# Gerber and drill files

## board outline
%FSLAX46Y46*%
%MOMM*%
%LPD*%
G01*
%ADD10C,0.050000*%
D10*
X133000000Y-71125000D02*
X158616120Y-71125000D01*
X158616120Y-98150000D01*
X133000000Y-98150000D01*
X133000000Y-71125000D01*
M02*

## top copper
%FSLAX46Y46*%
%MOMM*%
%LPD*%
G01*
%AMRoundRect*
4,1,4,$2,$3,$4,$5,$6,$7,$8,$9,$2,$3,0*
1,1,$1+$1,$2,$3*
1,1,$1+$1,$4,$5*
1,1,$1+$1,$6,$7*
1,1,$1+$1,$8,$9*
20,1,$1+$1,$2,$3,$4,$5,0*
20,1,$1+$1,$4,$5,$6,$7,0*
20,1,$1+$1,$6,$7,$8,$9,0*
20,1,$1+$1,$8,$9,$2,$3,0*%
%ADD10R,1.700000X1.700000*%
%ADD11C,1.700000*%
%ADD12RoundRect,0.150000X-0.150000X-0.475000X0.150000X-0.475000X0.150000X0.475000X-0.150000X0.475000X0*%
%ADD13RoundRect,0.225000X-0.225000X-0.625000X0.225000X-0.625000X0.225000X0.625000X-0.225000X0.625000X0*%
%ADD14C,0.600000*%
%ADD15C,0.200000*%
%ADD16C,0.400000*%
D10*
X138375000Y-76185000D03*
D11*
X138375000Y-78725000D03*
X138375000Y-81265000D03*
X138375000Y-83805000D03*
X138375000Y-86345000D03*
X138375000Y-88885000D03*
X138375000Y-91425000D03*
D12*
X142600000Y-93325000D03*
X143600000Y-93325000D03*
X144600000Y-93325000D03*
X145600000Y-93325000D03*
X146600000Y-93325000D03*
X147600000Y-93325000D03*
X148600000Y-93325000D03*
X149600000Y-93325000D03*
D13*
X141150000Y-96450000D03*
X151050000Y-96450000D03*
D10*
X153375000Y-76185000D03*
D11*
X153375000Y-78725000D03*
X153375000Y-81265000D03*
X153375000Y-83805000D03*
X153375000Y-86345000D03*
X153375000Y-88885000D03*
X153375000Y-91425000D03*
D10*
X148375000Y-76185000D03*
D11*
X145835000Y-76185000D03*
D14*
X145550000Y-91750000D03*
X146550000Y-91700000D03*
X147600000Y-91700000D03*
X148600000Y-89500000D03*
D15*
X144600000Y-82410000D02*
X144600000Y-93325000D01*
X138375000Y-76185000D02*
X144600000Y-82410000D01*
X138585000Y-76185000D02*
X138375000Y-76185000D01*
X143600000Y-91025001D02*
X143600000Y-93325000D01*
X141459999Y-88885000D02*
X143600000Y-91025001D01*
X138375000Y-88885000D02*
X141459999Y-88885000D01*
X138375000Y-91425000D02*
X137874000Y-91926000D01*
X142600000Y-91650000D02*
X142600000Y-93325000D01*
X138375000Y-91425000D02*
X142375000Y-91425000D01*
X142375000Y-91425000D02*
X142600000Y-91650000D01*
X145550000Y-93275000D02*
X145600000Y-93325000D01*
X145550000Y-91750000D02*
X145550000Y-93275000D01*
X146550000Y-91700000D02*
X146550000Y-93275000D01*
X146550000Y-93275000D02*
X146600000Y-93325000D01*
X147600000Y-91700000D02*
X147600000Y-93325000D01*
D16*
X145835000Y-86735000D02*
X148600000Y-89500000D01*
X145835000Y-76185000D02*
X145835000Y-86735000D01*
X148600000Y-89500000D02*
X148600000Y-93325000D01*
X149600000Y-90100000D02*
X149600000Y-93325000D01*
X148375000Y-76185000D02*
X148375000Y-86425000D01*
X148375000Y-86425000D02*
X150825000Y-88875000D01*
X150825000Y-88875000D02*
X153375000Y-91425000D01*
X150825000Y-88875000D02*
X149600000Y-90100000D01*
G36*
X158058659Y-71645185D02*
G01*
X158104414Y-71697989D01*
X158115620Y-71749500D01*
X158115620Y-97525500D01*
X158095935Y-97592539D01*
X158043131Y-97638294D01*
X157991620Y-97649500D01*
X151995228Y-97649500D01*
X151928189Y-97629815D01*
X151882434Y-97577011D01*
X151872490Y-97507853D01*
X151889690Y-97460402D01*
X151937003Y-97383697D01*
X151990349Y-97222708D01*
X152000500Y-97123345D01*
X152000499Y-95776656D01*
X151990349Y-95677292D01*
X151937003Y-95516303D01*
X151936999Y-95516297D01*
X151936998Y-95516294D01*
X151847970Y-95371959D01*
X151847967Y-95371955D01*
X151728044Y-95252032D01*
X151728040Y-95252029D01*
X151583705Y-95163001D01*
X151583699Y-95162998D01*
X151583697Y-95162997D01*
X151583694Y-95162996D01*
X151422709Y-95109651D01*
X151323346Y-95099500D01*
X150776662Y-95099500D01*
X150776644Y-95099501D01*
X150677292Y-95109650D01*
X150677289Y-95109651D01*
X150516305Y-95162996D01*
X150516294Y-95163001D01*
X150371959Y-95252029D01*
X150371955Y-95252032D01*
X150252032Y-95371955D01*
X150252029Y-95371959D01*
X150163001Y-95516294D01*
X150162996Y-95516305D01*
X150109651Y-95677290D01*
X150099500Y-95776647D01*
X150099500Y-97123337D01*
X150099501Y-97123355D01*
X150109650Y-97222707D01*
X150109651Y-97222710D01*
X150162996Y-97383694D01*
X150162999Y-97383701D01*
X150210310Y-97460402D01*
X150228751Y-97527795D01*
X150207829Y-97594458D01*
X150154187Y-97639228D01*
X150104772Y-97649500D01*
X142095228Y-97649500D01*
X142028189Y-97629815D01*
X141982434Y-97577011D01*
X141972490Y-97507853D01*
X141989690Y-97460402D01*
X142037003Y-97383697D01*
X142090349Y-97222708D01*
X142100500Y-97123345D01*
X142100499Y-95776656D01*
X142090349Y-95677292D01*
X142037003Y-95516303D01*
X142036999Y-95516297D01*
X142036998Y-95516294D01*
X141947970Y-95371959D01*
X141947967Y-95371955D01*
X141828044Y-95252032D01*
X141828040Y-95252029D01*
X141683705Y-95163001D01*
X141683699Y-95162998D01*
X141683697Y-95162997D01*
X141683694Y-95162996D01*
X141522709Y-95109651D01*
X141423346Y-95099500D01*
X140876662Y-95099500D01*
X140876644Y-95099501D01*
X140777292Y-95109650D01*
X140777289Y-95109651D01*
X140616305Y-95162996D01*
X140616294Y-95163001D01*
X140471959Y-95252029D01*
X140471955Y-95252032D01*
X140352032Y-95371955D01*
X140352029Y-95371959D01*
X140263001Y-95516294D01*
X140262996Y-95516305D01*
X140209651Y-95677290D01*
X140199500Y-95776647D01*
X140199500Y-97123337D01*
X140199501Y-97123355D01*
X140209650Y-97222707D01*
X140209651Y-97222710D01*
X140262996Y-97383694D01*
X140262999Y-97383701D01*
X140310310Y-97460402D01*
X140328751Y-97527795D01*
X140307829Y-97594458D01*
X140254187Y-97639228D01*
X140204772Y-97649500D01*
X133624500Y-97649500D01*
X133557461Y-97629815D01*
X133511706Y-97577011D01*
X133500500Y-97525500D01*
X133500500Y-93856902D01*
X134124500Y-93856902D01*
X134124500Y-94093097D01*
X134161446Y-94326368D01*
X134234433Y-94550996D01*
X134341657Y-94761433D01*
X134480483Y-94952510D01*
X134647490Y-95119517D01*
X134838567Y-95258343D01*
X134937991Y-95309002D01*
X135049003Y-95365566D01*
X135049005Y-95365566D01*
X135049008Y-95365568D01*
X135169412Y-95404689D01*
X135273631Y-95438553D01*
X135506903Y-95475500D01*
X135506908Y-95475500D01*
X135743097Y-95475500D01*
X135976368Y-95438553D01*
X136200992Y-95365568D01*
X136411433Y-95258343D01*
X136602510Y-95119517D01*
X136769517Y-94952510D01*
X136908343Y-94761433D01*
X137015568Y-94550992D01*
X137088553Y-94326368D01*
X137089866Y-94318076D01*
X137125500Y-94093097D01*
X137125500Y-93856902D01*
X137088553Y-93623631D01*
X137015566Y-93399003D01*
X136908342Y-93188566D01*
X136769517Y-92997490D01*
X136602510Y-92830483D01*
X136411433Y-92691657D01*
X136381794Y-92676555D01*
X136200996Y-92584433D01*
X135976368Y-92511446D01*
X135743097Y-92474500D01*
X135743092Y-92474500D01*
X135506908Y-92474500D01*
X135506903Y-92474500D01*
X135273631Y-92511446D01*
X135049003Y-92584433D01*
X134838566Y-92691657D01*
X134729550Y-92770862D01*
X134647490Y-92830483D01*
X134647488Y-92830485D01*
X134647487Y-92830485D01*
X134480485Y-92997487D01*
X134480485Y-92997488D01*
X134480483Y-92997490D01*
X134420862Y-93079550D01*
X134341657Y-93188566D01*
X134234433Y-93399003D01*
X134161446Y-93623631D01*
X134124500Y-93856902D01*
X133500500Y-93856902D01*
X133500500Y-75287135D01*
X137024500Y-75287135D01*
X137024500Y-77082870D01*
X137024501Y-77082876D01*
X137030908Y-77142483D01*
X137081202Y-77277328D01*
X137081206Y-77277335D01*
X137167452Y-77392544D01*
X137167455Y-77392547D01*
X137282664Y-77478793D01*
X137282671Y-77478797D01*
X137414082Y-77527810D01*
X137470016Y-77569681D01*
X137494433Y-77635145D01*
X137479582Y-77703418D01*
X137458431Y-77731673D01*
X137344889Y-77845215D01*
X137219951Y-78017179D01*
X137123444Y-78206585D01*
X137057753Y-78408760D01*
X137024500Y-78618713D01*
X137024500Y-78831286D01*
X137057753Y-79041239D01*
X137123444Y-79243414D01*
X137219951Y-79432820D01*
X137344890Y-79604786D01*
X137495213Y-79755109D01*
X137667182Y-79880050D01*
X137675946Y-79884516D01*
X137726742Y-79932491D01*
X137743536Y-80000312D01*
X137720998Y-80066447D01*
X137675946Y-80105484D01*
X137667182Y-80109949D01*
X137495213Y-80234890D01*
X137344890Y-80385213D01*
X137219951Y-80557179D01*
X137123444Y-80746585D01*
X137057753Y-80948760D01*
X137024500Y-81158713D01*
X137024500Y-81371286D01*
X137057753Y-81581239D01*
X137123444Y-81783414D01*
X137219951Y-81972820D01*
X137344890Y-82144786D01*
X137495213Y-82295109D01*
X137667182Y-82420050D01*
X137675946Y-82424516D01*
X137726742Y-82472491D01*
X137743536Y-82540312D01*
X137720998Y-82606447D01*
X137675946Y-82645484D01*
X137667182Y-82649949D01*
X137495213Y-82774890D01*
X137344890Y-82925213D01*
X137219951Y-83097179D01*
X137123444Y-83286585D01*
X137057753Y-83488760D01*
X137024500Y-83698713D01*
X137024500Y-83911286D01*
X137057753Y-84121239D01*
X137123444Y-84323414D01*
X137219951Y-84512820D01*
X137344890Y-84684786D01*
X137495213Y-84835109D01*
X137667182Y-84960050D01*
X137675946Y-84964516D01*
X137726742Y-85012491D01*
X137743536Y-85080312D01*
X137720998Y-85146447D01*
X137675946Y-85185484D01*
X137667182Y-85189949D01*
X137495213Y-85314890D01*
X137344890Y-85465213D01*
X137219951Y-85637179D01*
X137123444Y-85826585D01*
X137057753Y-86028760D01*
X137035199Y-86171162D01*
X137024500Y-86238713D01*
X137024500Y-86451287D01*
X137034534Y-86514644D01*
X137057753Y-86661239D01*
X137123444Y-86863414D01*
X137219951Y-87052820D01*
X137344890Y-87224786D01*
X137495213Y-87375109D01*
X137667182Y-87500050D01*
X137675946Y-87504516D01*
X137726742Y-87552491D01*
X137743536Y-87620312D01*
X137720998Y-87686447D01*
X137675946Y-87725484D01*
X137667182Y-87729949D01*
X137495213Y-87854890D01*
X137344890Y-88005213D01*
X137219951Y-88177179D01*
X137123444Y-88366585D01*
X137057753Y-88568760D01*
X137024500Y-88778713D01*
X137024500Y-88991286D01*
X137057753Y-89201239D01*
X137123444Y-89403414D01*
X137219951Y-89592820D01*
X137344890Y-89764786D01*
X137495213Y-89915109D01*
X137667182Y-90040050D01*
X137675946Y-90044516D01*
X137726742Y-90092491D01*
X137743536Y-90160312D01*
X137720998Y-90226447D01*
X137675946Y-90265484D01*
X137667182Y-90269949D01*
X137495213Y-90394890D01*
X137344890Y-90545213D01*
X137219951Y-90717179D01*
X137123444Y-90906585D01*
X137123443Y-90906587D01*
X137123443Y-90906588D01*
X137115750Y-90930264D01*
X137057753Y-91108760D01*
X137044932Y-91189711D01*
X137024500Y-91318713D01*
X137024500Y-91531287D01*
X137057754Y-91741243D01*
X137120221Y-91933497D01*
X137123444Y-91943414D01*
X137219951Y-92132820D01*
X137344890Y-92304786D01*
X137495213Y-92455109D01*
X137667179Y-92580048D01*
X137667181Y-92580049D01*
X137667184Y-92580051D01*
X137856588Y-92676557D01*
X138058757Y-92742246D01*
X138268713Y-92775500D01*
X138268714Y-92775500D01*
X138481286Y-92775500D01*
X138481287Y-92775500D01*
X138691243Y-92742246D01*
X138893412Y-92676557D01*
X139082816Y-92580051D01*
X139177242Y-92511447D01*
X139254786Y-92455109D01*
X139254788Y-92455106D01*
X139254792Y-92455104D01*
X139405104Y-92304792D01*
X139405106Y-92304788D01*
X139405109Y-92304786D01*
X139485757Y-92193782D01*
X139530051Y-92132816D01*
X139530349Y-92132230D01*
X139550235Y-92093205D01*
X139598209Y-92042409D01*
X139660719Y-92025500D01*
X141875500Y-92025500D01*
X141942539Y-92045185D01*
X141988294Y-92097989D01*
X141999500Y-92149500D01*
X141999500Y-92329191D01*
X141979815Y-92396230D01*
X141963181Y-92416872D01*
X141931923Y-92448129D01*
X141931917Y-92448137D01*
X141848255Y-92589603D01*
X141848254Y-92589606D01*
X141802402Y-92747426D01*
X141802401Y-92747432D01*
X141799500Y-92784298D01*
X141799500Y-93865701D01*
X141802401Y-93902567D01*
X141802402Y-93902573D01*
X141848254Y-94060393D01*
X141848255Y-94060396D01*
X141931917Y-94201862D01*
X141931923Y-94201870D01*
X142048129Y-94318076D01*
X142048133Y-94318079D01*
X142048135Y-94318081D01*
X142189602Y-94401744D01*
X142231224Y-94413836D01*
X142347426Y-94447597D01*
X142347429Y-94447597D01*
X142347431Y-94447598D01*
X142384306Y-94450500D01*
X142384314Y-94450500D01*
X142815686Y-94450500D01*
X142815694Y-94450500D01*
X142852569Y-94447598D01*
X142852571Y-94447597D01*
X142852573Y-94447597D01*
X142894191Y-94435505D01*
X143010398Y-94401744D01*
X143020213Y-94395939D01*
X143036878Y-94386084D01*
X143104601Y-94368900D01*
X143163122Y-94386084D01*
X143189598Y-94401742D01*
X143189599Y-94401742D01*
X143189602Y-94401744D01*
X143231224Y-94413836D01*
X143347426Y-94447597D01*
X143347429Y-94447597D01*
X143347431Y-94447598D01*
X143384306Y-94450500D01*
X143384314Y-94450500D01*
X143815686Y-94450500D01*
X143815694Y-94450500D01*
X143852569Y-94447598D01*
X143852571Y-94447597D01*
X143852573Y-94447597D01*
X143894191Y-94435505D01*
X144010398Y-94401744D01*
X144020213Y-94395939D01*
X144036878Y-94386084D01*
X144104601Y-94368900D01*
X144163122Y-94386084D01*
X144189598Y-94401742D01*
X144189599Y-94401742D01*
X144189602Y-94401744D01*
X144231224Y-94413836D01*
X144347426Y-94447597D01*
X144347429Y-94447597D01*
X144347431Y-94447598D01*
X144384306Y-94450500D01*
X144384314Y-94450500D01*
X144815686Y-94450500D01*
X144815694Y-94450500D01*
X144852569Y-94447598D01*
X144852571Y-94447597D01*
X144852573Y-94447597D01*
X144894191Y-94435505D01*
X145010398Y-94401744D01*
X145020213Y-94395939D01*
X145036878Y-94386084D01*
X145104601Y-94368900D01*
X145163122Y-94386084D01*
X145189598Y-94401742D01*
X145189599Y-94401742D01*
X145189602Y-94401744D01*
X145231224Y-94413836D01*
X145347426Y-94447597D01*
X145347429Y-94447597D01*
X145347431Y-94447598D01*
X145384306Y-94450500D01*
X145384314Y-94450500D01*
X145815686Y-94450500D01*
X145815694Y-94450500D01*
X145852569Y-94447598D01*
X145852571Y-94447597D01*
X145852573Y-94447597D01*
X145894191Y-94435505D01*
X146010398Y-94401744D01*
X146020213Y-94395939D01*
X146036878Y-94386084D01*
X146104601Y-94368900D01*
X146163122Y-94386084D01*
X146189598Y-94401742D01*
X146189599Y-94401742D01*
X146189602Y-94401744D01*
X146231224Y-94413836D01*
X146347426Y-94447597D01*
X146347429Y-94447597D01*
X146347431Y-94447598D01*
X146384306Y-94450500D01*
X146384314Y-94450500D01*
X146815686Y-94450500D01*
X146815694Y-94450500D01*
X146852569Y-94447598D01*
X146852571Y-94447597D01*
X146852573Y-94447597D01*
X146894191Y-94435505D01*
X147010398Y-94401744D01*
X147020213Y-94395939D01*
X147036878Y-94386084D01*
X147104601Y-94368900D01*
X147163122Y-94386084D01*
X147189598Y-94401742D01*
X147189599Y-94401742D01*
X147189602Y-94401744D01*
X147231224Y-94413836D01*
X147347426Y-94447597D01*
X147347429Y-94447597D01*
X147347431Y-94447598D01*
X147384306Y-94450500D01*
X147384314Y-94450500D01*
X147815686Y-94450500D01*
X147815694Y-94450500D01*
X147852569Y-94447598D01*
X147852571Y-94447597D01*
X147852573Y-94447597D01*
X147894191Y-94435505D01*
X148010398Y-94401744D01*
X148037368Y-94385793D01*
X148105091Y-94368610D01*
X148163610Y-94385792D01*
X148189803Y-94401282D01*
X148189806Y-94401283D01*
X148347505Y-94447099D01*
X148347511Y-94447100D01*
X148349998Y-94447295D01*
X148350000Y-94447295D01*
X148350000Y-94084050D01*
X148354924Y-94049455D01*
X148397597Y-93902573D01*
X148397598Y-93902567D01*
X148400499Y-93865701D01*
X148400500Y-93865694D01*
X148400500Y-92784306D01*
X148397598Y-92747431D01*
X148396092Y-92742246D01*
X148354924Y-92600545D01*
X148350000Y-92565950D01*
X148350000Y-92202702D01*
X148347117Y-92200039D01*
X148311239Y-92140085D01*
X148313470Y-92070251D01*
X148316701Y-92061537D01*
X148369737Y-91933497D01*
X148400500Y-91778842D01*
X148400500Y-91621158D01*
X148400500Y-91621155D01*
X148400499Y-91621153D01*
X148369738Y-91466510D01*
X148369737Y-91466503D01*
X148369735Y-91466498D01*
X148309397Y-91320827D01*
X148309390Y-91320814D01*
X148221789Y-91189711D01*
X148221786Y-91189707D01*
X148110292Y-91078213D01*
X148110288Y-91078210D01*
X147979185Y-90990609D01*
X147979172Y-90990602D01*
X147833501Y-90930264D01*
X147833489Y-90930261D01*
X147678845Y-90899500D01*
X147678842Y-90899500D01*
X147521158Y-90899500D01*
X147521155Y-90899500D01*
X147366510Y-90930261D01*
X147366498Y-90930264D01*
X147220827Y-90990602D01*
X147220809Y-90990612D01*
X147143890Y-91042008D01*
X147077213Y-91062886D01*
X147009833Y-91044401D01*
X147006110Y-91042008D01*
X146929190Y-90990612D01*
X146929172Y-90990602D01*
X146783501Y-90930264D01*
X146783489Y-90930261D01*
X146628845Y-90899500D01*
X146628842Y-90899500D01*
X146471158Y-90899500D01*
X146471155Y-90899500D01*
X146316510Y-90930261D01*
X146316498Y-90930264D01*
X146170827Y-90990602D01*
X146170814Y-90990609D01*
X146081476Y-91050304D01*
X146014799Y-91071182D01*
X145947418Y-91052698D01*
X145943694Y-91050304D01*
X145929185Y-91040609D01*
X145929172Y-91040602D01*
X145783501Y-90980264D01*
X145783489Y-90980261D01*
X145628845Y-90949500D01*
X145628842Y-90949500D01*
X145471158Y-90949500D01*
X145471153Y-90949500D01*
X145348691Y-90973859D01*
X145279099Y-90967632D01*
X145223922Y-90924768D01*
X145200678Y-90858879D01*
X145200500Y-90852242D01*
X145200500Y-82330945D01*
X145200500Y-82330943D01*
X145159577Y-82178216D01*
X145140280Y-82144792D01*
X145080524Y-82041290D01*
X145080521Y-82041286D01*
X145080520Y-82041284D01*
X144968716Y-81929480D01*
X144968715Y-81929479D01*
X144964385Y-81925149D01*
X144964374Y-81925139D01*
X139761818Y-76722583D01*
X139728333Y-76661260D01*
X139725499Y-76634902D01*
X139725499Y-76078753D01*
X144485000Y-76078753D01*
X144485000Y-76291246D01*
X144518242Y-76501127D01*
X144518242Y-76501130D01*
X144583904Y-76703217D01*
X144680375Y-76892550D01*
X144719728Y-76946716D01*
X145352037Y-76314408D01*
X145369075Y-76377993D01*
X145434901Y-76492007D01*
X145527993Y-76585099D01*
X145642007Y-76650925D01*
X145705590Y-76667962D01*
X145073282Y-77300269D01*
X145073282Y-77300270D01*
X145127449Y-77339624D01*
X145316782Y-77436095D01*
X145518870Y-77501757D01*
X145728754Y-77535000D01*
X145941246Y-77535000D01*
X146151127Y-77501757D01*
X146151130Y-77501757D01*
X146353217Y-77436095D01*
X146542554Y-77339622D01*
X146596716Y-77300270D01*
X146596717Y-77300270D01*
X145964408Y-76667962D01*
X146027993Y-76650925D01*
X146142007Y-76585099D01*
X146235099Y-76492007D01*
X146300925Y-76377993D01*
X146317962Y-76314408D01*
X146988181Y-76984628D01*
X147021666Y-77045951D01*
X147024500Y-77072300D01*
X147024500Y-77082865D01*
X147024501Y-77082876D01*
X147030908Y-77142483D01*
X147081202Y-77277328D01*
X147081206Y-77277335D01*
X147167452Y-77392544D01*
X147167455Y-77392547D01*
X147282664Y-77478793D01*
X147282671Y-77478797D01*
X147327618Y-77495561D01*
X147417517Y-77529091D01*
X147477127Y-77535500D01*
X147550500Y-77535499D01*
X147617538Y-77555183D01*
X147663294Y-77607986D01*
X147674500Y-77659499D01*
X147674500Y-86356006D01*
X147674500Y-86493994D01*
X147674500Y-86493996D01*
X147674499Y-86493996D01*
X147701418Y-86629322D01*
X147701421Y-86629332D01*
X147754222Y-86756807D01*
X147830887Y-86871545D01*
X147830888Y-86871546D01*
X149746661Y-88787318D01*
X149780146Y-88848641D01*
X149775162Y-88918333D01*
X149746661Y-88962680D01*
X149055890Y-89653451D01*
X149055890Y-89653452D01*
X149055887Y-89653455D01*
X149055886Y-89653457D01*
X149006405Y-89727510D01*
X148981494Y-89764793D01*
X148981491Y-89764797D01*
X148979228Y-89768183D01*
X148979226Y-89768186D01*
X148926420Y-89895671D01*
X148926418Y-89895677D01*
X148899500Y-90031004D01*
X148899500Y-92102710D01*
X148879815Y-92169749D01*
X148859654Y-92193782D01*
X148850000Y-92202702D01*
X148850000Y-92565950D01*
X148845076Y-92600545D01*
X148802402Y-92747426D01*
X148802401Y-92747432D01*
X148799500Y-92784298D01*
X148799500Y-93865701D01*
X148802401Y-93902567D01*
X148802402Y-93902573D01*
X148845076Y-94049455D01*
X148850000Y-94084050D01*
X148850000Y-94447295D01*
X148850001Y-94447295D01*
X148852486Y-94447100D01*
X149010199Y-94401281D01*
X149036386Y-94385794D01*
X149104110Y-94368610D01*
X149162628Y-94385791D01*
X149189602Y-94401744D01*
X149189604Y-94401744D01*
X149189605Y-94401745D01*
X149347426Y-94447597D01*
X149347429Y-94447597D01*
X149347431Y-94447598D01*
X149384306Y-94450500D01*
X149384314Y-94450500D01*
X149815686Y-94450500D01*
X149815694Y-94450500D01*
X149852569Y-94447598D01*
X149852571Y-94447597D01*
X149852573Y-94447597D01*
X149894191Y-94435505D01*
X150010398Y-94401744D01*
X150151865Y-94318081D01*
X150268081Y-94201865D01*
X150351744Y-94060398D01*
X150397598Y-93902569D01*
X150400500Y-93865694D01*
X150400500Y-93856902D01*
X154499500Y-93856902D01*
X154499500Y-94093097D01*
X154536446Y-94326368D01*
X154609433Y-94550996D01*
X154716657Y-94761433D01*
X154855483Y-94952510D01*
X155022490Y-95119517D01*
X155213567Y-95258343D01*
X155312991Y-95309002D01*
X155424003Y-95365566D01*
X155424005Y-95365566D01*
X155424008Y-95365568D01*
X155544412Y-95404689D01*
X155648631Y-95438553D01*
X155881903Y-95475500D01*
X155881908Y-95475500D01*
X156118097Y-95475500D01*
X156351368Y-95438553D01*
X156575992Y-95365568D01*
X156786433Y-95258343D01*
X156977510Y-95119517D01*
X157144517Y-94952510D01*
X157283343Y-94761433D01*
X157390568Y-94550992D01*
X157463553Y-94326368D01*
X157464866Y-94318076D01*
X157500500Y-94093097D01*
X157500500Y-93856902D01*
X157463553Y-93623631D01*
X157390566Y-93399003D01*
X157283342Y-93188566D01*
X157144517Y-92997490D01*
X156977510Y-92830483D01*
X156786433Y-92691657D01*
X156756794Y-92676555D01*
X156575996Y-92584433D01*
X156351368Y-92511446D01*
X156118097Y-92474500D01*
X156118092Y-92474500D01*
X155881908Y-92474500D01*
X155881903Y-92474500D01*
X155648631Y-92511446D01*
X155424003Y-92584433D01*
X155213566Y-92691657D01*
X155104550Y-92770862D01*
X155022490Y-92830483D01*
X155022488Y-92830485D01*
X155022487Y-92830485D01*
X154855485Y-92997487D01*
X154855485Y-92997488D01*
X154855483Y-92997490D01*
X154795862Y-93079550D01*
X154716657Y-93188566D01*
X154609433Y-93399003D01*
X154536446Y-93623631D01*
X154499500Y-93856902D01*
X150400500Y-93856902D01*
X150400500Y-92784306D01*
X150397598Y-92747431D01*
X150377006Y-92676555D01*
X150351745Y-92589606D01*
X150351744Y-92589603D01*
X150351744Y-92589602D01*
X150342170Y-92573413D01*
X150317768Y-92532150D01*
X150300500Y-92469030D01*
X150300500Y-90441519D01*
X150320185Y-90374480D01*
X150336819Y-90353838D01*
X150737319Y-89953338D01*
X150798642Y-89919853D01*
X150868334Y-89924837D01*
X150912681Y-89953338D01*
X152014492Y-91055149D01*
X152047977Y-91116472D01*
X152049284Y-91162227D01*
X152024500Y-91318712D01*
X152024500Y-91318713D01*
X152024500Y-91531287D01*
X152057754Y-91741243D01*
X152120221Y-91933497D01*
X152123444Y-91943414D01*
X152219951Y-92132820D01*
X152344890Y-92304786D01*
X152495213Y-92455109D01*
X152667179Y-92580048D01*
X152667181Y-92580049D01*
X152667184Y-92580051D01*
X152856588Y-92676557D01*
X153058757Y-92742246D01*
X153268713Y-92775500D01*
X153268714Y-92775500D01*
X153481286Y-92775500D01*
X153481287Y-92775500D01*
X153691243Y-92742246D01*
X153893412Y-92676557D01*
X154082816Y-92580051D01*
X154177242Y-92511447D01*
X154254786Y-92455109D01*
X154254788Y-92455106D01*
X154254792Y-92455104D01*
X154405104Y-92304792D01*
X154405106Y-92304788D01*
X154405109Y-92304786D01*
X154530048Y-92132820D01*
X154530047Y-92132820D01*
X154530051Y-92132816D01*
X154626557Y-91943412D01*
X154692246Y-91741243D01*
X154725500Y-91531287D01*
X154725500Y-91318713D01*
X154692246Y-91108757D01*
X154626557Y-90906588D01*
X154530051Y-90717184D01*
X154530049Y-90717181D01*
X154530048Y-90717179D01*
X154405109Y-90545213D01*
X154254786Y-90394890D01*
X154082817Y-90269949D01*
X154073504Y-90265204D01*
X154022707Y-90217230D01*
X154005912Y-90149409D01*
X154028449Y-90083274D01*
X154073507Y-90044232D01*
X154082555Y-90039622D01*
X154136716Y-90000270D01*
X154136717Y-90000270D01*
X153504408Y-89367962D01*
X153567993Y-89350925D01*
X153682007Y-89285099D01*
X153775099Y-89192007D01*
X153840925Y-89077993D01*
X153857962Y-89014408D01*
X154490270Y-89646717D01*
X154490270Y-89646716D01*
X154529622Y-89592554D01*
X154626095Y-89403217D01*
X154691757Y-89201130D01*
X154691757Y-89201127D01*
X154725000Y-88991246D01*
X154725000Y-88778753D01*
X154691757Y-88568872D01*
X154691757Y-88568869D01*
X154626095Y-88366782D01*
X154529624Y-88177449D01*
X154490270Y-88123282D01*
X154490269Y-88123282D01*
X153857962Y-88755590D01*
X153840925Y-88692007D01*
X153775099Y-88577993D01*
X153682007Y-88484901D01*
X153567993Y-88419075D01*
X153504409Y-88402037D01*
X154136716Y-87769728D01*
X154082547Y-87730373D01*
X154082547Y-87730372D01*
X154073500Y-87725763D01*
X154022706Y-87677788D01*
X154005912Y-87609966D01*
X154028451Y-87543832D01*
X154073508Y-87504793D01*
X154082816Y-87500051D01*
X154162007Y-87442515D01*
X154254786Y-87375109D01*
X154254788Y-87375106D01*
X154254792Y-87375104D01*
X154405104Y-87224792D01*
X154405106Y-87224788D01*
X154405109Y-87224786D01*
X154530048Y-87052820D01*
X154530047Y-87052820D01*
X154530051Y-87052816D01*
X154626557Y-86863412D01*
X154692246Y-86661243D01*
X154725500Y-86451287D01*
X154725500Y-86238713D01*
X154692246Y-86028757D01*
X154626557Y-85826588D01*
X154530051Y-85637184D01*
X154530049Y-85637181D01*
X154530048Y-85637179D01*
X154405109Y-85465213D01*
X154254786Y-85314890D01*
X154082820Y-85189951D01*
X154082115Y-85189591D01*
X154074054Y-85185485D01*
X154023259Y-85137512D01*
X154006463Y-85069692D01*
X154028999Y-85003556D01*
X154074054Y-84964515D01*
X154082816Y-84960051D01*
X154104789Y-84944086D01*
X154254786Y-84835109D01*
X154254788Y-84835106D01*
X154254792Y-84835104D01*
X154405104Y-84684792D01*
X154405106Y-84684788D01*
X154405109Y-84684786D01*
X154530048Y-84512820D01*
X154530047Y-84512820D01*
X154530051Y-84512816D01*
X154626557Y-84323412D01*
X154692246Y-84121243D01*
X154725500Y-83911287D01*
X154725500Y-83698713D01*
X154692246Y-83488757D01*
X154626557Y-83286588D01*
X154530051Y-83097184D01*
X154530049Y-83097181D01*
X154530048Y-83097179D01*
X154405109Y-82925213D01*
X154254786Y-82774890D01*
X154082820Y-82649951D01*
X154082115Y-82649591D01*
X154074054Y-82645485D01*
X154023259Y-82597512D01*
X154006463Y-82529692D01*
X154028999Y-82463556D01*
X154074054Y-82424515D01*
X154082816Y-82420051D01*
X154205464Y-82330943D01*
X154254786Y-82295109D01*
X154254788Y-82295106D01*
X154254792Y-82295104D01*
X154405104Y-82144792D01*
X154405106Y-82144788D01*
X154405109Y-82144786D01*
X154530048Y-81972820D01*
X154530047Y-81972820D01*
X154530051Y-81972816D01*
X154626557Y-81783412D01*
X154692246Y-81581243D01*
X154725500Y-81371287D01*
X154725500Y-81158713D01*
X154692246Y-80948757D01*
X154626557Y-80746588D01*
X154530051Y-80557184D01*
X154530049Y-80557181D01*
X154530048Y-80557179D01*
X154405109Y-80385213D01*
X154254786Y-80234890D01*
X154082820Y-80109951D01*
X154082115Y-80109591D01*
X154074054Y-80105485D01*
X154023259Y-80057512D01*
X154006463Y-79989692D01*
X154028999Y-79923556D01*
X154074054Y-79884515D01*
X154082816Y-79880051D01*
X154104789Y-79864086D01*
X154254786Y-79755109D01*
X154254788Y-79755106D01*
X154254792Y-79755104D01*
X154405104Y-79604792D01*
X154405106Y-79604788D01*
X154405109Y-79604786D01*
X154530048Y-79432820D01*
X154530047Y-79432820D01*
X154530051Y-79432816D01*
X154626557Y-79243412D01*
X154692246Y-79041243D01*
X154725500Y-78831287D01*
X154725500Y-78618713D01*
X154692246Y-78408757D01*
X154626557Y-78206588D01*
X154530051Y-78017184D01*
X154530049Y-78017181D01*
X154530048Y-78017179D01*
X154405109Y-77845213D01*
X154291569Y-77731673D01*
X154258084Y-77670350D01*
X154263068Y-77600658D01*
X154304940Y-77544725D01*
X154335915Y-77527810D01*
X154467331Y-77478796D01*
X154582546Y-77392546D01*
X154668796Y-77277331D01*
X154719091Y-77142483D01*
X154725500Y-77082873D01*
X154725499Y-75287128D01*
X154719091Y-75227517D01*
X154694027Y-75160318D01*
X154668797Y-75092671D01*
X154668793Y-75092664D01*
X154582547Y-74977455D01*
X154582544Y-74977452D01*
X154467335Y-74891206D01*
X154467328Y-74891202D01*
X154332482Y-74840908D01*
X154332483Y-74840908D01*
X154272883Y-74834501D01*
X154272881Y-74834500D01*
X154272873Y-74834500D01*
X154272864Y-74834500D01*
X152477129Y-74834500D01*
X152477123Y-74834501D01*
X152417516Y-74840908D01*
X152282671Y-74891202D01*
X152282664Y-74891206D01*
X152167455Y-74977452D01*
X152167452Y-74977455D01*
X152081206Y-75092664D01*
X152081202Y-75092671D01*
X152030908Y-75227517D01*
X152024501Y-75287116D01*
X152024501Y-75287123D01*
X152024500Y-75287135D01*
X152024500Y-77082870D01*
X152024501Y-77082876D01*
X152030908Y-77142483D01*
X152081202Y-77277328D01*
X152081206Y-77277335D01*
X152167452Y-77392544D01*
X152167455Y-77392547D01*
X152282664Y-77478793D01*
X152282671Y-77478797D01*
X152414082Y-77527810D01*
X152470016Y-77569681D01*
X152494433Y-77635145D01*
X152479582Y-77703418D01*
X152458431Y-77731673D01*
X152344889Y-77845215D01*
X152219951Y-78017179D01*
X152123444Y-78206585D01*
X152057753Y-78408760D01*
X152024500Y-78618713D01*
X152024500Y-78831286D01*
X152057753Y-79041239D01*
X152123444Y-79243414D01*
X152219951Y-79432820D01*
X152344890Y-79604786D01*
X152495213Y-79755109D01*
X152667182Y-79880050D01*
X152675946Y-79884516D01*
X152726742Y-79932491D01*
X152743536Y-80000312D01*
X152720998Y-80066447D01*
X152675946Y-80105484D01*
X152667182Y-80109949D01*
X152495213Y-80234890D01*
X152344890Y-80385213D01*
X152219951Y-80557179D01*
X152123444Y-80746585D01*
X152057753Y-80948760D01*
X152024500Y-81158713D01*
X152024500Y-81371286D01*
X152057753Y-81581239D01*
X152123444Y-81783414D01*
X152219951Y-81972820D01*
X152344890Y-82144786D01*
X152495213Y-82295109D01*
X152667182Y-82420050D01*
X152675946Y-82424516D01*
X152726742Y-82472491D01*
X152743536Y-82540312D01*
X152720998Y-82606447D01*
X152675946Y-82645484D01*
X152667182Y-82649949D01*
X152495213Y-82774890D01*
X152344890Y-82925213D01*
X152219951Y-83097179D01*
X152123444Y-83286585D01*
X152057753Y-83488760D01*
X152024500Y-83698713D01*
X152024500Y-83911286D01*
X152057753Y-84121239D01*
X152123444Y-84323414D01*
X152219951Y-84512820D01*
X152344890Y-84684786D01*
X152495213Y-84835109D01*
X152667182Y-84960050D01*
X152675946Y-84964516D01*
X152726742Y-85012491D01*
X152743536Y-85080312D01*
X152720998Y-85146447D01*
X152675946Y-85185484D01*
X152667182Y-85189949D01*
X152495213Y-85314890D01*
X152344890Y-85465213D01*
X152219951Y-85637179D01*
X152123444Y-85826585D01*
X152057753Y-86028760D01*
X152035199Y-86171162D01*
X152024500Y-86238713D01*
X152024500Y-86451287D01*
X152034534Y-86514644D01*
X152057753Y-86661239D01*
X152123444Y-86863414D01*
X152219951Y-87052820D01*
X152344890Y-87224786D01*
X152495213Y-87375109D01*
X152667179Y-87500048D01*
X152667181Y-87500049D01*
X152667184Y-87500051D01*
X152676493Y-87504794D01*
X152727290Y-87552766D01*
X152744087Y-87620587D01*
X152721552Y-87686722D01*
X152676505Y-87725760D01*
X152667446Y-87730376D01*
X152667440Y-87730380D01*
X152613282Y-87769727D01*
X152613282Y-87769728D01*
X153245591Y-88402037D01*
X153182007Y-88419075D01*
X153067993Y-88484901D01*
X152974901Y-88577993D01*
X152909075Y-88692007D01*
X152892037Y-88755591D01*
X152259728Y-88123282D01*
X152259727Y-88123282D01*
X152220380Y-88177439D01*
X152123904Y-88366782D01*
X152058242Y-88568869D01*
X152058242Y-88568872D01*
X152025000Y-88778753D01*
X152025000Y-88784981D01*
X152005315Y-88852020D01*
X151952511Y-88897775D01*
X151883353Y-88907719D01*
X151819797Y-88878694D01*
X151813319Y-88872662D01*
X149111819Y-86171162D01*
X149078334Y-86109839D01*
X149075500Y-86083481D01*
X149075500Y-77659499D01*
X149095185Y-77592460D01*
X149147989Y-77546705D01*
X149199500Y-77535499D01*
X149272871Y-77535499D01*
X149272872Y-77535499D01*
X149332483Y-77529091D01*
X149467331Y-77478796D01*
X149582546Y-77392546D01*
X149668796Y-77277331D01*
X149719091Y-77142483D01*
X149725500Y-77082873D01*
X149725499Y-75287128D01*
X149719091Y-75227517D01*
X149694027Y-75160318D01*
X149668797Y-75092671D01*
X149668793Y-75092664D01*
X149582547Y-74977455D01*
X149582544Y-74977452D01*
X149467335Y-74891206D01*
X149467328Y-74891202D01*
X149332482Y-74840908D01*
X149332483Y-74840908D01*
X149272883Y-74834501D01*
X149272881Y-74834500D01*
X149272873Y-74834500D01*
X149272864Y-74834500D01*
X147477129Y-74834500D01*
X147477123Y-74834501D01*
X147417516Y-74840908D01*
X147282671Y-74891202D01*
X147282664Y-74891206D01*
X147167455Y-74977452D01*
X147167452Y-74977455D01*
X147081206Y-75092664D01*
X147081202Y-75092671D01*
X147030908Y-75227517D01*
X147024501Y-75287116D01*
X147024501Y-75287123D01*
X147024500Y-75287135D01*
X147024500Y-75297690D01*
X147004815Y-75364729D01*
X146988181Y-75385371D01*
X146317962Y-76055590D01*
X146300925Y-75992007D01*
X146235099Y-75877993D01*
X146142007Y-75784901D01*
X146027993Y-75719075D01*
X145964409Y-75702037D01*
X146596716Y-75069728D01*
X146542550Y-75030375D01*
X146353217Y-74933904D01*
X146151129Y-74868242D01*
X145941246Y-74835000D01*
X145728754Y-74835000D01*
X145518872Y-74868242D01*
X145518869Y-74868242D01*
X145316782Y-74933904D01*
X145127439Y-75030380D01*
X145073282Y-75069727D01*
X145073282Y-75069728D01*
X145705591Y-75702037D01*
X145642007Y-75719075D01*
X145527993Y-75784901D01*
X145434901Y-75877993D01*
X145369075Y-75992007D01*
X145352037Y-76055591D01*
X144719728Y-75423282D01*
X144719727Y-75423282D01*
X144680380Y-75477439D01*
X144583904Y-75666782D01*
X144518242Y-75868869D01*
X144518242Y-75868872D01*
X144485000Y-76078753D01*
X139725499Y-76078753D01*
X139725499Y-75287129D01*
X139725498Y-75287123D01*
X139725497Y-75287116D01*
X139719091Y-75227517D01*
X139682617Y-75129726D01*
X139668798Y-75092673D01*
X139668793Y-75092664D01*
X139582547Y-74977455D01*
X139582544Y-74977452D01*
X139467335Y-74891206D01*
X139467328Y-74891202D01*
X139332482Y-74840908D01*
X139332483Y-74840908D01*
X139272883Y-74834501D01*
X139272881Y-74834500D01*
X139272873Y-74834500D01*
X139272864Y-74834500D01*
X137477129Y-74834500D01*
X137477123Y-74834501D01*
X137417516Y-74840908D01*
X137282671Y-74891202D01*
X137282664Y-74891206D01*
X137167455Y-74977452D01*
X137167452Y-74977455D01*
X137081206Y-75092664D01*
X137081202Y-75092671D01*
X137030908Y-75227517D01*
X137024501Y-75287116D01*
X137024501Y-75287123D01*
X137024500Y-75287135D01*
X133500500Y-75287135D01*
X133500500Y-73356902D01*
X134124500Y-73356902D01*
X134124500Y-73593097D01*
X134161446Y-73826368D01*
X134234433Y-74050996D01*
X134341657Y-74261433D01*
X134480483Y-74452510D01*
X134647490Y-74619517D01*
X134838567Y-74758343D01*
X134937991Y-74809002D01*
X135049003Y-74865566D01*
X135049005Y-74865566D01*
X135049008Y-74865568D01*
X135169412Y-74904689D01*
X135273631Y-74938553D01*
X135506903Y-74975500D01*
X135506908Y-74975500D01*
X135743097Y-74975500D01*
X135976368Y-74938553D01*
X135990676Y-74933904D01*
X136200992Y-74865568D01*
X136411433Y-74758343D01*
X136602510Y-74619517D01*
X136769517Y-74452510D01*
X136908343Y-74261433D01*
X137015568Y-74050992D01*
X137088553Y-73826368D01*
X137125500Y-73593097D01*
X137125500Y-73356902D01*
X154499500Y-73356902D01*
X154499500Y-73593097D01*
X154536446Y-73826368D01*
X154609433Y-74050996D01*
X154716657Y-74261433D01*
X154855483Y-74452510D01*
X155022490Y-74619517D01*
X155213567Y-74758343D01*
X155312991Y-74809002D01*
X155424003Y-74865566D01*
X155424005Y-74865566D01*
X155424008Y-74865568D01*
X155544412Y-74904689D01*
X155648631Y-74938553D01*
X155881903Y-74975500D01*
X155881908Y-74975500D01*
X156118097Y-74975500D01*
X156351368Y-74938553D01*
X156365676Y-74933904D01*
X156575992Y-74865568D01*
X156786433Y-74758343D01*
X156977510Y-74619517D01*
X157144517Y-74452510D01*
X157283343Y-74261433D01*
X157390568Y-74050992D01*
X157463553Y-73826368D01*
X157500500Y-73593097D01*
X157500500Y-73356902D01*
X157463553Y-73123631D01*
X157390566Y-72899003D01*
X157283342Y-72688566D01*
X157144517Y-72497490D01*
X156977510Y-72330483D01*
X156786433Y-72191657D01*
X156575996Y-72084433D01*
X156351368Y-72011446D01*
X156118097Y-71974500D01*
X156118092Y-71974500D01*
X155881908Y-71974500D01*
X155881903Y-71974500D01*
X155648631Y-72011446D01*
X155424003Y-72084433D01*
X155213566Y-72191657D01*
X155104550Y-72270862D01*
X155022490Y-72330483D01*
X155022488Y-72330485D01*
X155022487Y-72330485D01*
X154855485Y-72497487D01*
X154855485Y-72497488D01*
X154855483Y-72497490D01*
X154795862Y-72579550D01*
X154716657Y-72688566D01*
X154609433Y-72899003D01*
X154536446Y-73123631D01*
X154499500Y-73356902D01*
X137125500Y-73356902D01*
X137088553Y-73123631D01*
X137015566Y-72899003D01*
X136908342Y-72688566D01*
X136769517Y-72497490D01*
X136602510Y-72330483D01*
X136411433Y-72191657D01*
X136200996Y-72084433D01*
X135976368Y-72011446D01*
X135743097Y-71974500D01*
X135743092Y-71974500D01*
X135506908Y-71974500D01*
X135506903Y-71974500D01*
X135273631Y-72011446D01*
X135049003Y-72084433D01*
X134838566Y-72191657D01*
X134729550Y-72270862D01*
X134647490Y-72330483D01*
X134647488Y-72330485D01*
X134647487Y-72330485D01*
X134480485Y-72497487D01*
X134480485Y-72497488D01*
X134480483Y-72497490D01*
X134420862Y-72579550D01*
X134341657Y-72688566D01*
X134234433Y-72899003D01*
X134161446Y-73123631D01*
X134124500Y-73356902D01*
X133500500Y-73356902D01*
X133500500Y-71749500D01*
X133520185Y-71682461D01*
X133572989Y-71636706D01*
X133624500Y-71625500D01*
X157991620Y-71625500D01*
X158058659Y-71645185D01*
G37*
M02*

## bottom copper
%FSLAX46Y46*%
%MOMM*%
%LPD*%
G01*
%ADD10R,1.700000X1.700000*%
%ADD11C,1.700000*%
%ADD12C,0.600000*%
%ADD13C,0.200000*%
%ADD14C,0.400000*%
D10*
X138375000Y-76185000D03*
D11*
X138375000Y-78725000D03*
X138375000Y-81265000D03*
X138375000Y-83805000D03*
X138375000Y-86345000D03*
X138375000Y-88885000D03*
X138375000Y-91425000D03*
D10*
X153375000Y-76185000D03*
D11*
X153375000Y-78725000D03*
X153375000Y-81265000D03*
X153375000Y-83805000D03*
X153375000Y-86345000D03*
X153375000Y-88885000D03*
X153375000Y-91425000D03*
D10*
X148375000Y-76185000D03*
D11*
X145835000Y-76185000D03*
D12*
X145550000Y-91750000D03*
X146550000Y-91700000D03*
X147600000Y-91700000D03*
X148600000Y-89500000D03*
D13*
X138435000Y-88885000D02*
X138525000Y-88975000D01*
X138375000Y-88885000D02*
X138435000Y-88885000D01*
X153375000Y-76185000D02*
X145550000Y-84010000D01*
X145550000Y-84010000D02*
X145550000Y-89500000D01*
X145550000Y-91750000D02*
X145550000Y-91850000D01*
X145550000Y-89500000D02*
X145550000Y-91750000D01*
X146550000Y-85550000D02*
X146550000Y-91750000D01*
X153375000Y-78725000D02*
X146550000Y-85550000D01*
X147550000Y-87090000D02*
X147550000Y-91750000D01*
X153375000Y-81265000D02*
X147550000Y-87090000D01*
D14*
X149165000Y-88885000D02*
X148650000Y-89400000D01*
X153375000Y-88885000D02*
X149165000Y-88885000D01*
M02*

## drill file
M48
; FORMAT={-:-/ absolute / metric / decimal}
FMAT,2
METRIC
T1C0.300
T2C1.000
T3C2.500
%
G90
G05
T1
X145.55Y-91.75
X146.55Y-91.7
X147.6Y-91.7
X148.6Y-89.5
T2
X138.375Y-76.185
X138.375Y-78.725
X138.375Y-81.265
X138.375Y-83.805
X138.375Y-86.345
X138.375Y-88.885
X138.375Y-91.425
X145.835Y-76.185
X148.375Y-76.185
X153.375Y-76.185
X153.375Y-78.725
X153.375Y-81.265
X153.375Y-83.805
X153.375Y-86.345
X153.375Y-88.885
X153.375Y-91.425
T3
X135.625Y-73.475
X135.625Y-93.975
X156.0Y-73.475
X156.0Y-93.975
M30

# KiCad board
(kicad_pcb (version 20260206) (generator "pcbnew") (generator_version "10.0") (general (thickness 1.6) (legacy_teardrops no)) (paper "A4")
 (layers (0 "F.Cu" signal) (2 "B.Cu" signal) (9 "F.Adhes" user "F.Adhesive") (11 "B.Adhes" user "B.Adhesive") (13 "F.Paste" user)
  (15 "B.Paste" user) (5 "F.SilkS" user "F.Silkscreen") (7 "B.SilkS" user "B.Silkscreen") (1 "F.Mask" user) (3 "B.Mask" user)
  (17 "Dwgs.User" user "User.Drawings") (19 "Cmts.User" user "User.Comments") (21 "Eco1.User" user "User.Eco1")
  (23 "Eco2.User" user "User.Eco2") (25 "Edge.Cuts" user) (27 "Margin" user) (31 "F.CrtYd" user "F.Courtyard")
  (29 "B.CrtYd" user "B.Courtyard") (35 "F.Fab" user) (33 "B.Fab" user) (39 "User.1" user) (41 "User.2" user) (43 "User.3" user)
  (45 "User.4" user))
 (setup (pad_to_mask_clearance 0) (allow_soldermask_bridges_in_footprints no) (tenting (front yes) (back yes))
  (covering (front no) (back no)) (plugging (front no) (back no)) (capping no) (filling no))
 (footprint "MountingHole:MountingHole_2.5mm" (layer "F.Cu") (at 135.625 73.475)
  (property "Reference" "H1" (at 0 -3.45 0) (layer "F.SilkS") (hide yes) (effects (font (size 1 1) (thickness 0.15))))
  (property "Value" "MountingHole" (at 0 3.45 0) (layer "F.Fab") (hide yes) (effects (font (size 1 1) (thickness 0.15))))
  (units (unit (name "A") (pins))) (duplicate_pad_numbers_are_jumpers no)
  (pad "" np_thru_hole circle (at 0 0) (size 2.5 2.5) (drill 2.5) (layers "*.Cu" "*.Mask")))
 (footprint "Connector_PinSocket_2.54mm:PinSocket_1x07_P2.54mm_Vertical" (layer "F.Cu") (at 138.375 76.185)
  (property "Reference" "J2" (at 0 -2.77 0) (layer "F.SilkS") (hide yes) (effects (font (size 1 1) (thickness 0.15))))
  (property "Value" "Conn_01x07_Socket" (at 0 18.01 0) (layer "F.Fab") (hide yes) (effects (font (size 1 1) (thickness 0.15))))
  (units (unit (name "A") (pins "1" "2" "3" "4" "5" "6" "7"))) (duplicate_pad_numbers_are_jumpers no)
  (pad "1" thru_hole rect (at 0 0) (size 1.7 1.7) (drill 1) (layers "*.Cu" "*.Mask") (remove_unused_layers no) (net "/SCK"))
  (pad "2" thru_hole circle (at 0 2.54) (size 1.7 1.7) (drill 1) (layers "*.Cu" "*.Mask") (remove_unused_layers no)
   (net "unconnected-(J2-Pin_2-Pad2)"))
  (pad "3" thru_hole circle (at 0 5.08) (size 1.7 1.7) (drill 1) (layers "*.Cu" "*.Mask") (remove_unused_layers no)
   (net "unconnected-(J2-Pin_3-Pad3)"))
  (pad "4" thru_hole circle (at 0 7.62) (size 1.7 1.7) (drill 1) (layers "*.Cu" "*.Mask") (remove_unused_layers no)
   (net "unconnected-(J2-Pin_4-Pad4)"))
  (pad "5" thru_hole circle (at 0 10.16) (size 1.7 1.7) (drill 1) (layers "*.Cu" "*.Mask") (remove_unused_layers no)
   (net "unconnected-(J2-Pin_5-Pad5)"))
  (pad "6" thru_hole circle (at 0 12.7) (size 1.7 1.7) (drill 1) (layers "*.Cu" "*.Mask") (remove_unused_layers no) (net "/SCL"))
  (pad "7" thru_hole circle (at 0 15.24) (size 1.7 1.7) (drill 1) (layers "*.Cu" "*.Mask") (remove_unused_layers no) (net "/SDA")))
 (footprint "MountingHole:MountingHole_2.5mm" (layer "F.Cu") (at 156.125 93.975)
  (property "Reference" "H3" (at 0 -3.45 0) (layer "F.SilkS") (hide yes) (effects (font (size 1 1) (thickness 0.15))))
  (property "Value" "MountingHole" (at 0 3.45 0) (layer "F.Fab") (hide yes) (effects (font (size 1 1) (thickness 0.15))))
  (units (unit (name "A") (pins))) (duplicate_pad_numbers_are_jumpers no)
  (pad "" np_thru_hole circle (at -0.125 0) (size 2.5 2.5) (drill 2.5) (layers "*.Cu" "*.Mask")))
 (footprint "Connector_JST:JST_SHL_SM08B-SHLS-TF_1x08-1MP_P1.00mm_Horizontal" (layer "F.Cu") (at 146.1 95)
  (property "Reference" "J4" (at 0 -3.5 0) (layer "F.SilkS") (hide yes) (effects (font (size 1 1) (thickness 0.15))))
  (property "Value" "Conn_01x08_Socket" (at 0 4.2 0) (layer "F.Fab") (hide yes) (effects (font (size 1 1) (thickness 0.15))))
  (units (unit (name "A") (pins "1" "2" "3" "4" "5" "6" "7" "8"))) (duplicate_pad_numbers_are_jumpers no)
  (pad "1" smd roundrect (at -3.5 -1.675) (size 0.6 1.25) (layers "F.Cu" "F.Mask" "F.Paste") (roundrect_rratio 0.25) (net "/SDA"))
  (pad "2" smd roundrect (at -2.5 -1.675) (size 0.6 1.25) (layers "F.Cu" "F.Mask" "F.Paste") (roundrect_rratio 0.25) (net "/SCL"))
  (pad "3" smd roundrect (at -1.5 -1.675) (size 0.6 1.25) (layers "F.Cu" "F.Mask" "F.Paste") (roundrect_rratio 0.25) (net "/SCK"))
  (pad "4" smd roundrect (at -0.5 -1.675) (size 0.6 1.25) (layers "F.Cu" "F.Mask" "F.Paste") (roundrect_rratio 0.25) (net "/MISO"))
  (pad "5" smd roundrect (at 0.5 -1.675) (size 0.6 1.25) (layers "F.Cu" "F.Mask" "F.Paste") (roundrect_rratio 0.25) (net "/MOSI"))
  (pad "6" smd roundrect (at 1.5 -1.675) (size 0.6 1.25) (layers "F.Cu" "F.Mask" "F.Paste") (roundrect_rratio 0.25) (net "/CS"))
  (pad "7" smd roundrect (at 2.5 -1.675) (size 0.6 1.25) (layers "F.Cu" "F.Mask" "F.Paste") (roundrect_rratio 0.25) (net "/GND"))
  (pad "8" smd roundrect (at 3.5 -1.675) (size 0.6 1.25) (layers "F.Cu" "F.Mask" "F.Paste") (roundrect_rratio 0.25) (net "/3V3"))
  (pad "MP" smd roundrect (at -4.95 1.45) (size 0.9 1.7) (layers "F.Cu" "F.Mask" "F.Paste") (roundrect_rratio 0.25))
  (pad "MP" smd roundrect (at 4.95 1.45) (size 0.9 1.7) (layers "F.Cu" "F.Mask" "F.Paste") (roundrect_rratio 0.25)))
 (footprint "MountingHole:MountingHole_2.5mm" (layer "F.Cu") (at 156.125 73.475)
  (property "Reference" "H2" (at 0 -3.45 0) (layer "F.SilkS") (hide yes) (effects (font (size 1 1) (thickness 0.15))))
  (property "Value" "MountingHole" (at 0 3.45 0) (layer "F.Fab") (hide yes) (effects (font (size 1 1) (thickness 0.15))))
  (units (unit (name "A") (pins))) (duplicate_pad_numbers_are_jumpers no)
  (pad "" np_thru_hole circle (at -0.125 0) (size 2.5 2.5) (drill 2.5) (layers "*.Cu" "*.Mask")))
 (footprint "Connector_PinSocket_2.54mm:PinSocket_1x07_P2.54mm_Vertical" (layer "F.Cu") (at 153.375 76.185)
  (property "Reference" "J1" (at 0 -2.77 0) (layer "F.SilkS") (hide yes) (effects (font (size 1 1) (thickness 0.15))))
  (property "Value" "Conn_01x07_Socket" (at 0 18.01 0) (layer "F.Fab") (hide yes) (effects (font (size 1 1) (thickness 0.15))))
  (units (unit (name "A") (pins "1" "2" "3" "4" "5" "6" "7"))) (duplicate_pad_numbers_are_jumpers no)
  (pad "1" thru_hole rect (at 0 0) (size 1.7 1.7) (drill 1) (layers "*.Cu" "*.Mask") (remove_unused_layers no) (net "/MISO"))
  (pad "2" thru_hole circle (at 0 2.54) (size 1.7 1.7) (drill 1) (layers "*.Cu" "*.Mask") (remove_unused_layers no) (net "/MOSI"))
  (pad "3" thru_hole circle (at 0 5.08) (size 1.7 1.7) (drill 1) (layers "*.Cu" "*.Mask") (remove_unused_layers no) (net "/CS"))
  (pad "4" thru_hole circle (at 0 7.62) (size 1.7 1.7) (drill 1) (layers "*.Cu" "*.Mask") (remove_unused_layers no)
   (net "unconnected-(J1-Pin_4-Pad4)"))
  (pad "5" thru_hole circle (at 0 10.16) (size 1.7 1.7) (drill 1) (layers "*.Cu" "*.Mask") (remove_unused_layers no)
   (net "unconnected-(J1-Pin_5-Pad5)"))
  (pad "6" thru_hole circle (at 0 12.7) (size 1.7 1.7) (drill 1) (layers "*.Cu" "*.Mask") (remove_unused_layers no) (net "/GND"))
  (pad "7" thru_hole circle (at 0 15.24) (size 1.7 1.7) (drill 1) (layers "*.Cu" "*.Mask") (remove_unused_layers no) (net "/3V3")))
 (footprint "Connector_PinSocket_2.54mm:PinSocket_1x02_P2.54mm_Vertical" (layer "F.Cu") (at 148.375 76.185 -90)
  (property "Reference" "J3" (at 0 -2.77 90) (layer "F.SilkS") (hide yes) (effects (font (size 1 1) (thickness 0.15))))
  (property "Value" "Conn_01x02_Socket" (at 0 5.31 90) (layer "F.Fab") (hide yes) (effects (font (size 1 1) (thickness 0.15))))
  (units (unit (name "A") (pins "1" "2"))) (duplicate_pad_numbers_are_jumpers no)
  (pad "1" thru_hole rect (at 0 0 270) (size 1.7 1.7) (drill 1) (layers "*.Cu" "*.Mask") (remove_unused_layers no) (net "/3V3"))
  (pad "2" thru_hole circle (at 0 2.54 270) (size 1.7 1.7) (drill 1) (layers "*.Cu" "*.Mask") (remove_unused_layers no) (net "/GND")))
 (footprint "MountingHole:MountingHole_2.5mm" (layer "F.Cu") (at 135.625 93.975)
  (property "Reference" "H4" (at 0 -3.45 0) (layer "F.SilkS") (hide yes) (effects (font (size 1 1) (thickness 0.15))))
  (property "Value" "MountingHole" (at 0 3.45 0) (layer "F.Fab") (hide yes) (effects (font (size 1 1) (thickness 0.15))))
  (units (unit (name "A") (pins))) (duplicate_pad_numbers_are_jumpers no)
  (pad "" np_thru_hole circle (at 0 0) (size 2.5 2.5) (drill 2.5) (layers "*.Cu" "*.Mask")))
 (gr_rect (start 133 71.125) (end 158.61612 98.15) (stroke (width 0.05) (type default)) (fill no) (layer "Edge.Cuts"))
 (segment (start 144.6 82.41) (end 144.6 93.325) (width 0.2) (layer "F.Cu") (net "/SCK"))
 (segment (start 138.375 76.185) (end 144.6 82.41) (width 0.2) (layer "F.Cu") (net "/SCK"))
 (segment (start 138.585 76.185) (end 138.375 76.185) (width 0.2) (layer "F.Cu") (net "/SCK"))
 (segment (start 143.6 91.025001) (end 143.6 93.325) (width 0.2) (layer "F.Cu") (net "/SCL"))
 (segment (start 141.459999 88.885) (end 143.6 91.025001) (width 0.2) (layer "F.Cu") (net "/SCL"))
 (segment (start 138.375 88.885) (end 141.459999 88.885) (width 0.2) (layer "F.Cu") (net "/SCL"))
 (segment (start 138.435 88.885) (end 138.525 88.975) (width 0.2) (layer "B.Cu") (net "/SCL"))
 (segment (start 138.375 88.885) (end 138.435 88.885) (width 0.2) (layer "B.Cu") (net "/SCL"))
 (segment (start 138.375 91.425) (end 137.874 91.926) (width 0.2) (layer "F.Cu") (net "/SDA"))
 (segment (start 142.6 91.65) (end 142.6 93.325) (width 0.2) (layer "F.Cu") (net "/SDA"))
 (segment (start 138.375 91.425) (end 142.375 91.425) (width 0.2) (layer "F.Cu") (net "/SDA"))
 (segment (start 142.375 91.425) (end 142.6 91.65) (width 0.2) (layer "F.Cu") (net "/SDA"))
 (segment (start 145.55 93.275) (end 145.6 93.325) (width 0.2) (layer "F.Cu") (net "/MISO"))
 (segment (start 145.55 91.75) (end 145.55 93.275) (width 0.2) (layer "F.Cu") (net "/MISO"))
 (via (at 145.55 91.75) (size 0.6) (drill 0.3) (layers "F.Cu" "B.Cu") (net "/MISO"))
 (segment (start 153.375 76.185) (end 145.55 84.01) (width 0.2) (layer "B.Cu") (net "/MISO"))
 (segment (start 145.55 84.01) (end 145.55 89.5) (width 0.2) (layer "B.Cu") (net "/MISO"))
 (segment (start 145.55 91.75) (end 145.55 91.85) (width 0.2) (layer "B.Cu") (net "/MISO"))
 (segment (start 145.55 89.5) (end 145.55 91.75) (width 0.2) (layer "B.Cu") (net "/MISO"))
 (segment (start 146.55 91.7) (end 146.55 93.275) (width 0.2) (layer "F.Cu") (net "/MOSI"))
 (segment (start 146.55 93.275) (end 146.6 93.325) (width 0.2) (layer "F.Cu") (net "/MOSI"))
 (via (at 146.55 91.7) (size 0.6) (drill 0.3) (layers "F.Cu" "B.Cu") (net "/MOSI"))
 (segment (start 146.55 85.55) (end 146.55 91.75) (width 0.2) (layer "B.Cu") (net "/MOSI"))
 (segment (start 153.375 78.725) (end 146.55 85.55) (width 0.2) (layer "B.Cu") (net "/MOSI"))
 (segment (start 147.6 91.7) (end 147.6 93.325) (width 0.2) (layer "F.Cu") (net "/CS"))
 (via (at 147.6 91.7) (size 0.6) (drill 0.3) (layers "F.Cu" "B.Cu") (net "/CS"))
 (segment (start 147.55 87.09) (end 147.55 91.75) (width 0.2) (layer "B.Cu") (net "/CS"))
 (segment (start 153.375 81.265) (end 147.55 87.09) (width 0.2) (layer "B.Cu") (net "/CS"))
 (segment (start 145.835 86.735) (end 148.6 89.5) (width 0.4) (layer "F.Cu") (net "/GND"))
 (segment (start 145.835 76.185) (end 145.835 86.735) (width 0.4) (layer "F.Cu") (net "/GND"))
 (segment (start 148.6 89.5) (end 148.6 93.325) (width 0.4) (layer "F.Cu") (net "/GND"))
 (via (at 148.6 89.5) (size 0.6) (drill 0.3) (layers "F.Cu" "B.Cu") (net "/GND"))
 (segment (start 149.165 88.885) (end 148.65 89.4) (width 0.4) (layer "B.Cu") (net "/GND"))
 (segment (start 153.375 88.885) (end 149.165 88.885) (width 0.4) (layer "B.Cu") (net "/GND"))
 (segment (start 149.6 90.1) (end 149.6 93.325) (width 0.4) (layer "F.Cu") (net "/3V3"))
 (segment (start 148.375 76.185) (end 148.375 86.425) (width 0.4) (layer "F.Cu") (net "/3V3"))
 (segment (start 148.375 86.425) (end 150.825 88.875) (width 0.4) (layer "F.Cu") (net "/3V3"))
 (segment (start 150.825 88.875) (end 153.375 91.425) (width 0.4) (layer "F.Cu") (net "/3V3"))
 (segment (start 150.825 88.875) (end 149.6 90.1) (width 0.4) (layer "F.Cu") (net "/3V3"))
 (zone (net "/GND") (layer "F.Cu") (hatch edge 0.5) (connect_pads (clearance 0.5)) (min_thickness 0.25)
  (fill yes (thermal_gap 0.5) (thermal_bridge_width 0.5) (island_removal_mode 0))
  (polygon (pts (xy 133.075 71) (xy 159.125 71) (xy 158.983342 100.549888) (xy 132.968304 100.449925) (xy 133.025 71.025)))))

